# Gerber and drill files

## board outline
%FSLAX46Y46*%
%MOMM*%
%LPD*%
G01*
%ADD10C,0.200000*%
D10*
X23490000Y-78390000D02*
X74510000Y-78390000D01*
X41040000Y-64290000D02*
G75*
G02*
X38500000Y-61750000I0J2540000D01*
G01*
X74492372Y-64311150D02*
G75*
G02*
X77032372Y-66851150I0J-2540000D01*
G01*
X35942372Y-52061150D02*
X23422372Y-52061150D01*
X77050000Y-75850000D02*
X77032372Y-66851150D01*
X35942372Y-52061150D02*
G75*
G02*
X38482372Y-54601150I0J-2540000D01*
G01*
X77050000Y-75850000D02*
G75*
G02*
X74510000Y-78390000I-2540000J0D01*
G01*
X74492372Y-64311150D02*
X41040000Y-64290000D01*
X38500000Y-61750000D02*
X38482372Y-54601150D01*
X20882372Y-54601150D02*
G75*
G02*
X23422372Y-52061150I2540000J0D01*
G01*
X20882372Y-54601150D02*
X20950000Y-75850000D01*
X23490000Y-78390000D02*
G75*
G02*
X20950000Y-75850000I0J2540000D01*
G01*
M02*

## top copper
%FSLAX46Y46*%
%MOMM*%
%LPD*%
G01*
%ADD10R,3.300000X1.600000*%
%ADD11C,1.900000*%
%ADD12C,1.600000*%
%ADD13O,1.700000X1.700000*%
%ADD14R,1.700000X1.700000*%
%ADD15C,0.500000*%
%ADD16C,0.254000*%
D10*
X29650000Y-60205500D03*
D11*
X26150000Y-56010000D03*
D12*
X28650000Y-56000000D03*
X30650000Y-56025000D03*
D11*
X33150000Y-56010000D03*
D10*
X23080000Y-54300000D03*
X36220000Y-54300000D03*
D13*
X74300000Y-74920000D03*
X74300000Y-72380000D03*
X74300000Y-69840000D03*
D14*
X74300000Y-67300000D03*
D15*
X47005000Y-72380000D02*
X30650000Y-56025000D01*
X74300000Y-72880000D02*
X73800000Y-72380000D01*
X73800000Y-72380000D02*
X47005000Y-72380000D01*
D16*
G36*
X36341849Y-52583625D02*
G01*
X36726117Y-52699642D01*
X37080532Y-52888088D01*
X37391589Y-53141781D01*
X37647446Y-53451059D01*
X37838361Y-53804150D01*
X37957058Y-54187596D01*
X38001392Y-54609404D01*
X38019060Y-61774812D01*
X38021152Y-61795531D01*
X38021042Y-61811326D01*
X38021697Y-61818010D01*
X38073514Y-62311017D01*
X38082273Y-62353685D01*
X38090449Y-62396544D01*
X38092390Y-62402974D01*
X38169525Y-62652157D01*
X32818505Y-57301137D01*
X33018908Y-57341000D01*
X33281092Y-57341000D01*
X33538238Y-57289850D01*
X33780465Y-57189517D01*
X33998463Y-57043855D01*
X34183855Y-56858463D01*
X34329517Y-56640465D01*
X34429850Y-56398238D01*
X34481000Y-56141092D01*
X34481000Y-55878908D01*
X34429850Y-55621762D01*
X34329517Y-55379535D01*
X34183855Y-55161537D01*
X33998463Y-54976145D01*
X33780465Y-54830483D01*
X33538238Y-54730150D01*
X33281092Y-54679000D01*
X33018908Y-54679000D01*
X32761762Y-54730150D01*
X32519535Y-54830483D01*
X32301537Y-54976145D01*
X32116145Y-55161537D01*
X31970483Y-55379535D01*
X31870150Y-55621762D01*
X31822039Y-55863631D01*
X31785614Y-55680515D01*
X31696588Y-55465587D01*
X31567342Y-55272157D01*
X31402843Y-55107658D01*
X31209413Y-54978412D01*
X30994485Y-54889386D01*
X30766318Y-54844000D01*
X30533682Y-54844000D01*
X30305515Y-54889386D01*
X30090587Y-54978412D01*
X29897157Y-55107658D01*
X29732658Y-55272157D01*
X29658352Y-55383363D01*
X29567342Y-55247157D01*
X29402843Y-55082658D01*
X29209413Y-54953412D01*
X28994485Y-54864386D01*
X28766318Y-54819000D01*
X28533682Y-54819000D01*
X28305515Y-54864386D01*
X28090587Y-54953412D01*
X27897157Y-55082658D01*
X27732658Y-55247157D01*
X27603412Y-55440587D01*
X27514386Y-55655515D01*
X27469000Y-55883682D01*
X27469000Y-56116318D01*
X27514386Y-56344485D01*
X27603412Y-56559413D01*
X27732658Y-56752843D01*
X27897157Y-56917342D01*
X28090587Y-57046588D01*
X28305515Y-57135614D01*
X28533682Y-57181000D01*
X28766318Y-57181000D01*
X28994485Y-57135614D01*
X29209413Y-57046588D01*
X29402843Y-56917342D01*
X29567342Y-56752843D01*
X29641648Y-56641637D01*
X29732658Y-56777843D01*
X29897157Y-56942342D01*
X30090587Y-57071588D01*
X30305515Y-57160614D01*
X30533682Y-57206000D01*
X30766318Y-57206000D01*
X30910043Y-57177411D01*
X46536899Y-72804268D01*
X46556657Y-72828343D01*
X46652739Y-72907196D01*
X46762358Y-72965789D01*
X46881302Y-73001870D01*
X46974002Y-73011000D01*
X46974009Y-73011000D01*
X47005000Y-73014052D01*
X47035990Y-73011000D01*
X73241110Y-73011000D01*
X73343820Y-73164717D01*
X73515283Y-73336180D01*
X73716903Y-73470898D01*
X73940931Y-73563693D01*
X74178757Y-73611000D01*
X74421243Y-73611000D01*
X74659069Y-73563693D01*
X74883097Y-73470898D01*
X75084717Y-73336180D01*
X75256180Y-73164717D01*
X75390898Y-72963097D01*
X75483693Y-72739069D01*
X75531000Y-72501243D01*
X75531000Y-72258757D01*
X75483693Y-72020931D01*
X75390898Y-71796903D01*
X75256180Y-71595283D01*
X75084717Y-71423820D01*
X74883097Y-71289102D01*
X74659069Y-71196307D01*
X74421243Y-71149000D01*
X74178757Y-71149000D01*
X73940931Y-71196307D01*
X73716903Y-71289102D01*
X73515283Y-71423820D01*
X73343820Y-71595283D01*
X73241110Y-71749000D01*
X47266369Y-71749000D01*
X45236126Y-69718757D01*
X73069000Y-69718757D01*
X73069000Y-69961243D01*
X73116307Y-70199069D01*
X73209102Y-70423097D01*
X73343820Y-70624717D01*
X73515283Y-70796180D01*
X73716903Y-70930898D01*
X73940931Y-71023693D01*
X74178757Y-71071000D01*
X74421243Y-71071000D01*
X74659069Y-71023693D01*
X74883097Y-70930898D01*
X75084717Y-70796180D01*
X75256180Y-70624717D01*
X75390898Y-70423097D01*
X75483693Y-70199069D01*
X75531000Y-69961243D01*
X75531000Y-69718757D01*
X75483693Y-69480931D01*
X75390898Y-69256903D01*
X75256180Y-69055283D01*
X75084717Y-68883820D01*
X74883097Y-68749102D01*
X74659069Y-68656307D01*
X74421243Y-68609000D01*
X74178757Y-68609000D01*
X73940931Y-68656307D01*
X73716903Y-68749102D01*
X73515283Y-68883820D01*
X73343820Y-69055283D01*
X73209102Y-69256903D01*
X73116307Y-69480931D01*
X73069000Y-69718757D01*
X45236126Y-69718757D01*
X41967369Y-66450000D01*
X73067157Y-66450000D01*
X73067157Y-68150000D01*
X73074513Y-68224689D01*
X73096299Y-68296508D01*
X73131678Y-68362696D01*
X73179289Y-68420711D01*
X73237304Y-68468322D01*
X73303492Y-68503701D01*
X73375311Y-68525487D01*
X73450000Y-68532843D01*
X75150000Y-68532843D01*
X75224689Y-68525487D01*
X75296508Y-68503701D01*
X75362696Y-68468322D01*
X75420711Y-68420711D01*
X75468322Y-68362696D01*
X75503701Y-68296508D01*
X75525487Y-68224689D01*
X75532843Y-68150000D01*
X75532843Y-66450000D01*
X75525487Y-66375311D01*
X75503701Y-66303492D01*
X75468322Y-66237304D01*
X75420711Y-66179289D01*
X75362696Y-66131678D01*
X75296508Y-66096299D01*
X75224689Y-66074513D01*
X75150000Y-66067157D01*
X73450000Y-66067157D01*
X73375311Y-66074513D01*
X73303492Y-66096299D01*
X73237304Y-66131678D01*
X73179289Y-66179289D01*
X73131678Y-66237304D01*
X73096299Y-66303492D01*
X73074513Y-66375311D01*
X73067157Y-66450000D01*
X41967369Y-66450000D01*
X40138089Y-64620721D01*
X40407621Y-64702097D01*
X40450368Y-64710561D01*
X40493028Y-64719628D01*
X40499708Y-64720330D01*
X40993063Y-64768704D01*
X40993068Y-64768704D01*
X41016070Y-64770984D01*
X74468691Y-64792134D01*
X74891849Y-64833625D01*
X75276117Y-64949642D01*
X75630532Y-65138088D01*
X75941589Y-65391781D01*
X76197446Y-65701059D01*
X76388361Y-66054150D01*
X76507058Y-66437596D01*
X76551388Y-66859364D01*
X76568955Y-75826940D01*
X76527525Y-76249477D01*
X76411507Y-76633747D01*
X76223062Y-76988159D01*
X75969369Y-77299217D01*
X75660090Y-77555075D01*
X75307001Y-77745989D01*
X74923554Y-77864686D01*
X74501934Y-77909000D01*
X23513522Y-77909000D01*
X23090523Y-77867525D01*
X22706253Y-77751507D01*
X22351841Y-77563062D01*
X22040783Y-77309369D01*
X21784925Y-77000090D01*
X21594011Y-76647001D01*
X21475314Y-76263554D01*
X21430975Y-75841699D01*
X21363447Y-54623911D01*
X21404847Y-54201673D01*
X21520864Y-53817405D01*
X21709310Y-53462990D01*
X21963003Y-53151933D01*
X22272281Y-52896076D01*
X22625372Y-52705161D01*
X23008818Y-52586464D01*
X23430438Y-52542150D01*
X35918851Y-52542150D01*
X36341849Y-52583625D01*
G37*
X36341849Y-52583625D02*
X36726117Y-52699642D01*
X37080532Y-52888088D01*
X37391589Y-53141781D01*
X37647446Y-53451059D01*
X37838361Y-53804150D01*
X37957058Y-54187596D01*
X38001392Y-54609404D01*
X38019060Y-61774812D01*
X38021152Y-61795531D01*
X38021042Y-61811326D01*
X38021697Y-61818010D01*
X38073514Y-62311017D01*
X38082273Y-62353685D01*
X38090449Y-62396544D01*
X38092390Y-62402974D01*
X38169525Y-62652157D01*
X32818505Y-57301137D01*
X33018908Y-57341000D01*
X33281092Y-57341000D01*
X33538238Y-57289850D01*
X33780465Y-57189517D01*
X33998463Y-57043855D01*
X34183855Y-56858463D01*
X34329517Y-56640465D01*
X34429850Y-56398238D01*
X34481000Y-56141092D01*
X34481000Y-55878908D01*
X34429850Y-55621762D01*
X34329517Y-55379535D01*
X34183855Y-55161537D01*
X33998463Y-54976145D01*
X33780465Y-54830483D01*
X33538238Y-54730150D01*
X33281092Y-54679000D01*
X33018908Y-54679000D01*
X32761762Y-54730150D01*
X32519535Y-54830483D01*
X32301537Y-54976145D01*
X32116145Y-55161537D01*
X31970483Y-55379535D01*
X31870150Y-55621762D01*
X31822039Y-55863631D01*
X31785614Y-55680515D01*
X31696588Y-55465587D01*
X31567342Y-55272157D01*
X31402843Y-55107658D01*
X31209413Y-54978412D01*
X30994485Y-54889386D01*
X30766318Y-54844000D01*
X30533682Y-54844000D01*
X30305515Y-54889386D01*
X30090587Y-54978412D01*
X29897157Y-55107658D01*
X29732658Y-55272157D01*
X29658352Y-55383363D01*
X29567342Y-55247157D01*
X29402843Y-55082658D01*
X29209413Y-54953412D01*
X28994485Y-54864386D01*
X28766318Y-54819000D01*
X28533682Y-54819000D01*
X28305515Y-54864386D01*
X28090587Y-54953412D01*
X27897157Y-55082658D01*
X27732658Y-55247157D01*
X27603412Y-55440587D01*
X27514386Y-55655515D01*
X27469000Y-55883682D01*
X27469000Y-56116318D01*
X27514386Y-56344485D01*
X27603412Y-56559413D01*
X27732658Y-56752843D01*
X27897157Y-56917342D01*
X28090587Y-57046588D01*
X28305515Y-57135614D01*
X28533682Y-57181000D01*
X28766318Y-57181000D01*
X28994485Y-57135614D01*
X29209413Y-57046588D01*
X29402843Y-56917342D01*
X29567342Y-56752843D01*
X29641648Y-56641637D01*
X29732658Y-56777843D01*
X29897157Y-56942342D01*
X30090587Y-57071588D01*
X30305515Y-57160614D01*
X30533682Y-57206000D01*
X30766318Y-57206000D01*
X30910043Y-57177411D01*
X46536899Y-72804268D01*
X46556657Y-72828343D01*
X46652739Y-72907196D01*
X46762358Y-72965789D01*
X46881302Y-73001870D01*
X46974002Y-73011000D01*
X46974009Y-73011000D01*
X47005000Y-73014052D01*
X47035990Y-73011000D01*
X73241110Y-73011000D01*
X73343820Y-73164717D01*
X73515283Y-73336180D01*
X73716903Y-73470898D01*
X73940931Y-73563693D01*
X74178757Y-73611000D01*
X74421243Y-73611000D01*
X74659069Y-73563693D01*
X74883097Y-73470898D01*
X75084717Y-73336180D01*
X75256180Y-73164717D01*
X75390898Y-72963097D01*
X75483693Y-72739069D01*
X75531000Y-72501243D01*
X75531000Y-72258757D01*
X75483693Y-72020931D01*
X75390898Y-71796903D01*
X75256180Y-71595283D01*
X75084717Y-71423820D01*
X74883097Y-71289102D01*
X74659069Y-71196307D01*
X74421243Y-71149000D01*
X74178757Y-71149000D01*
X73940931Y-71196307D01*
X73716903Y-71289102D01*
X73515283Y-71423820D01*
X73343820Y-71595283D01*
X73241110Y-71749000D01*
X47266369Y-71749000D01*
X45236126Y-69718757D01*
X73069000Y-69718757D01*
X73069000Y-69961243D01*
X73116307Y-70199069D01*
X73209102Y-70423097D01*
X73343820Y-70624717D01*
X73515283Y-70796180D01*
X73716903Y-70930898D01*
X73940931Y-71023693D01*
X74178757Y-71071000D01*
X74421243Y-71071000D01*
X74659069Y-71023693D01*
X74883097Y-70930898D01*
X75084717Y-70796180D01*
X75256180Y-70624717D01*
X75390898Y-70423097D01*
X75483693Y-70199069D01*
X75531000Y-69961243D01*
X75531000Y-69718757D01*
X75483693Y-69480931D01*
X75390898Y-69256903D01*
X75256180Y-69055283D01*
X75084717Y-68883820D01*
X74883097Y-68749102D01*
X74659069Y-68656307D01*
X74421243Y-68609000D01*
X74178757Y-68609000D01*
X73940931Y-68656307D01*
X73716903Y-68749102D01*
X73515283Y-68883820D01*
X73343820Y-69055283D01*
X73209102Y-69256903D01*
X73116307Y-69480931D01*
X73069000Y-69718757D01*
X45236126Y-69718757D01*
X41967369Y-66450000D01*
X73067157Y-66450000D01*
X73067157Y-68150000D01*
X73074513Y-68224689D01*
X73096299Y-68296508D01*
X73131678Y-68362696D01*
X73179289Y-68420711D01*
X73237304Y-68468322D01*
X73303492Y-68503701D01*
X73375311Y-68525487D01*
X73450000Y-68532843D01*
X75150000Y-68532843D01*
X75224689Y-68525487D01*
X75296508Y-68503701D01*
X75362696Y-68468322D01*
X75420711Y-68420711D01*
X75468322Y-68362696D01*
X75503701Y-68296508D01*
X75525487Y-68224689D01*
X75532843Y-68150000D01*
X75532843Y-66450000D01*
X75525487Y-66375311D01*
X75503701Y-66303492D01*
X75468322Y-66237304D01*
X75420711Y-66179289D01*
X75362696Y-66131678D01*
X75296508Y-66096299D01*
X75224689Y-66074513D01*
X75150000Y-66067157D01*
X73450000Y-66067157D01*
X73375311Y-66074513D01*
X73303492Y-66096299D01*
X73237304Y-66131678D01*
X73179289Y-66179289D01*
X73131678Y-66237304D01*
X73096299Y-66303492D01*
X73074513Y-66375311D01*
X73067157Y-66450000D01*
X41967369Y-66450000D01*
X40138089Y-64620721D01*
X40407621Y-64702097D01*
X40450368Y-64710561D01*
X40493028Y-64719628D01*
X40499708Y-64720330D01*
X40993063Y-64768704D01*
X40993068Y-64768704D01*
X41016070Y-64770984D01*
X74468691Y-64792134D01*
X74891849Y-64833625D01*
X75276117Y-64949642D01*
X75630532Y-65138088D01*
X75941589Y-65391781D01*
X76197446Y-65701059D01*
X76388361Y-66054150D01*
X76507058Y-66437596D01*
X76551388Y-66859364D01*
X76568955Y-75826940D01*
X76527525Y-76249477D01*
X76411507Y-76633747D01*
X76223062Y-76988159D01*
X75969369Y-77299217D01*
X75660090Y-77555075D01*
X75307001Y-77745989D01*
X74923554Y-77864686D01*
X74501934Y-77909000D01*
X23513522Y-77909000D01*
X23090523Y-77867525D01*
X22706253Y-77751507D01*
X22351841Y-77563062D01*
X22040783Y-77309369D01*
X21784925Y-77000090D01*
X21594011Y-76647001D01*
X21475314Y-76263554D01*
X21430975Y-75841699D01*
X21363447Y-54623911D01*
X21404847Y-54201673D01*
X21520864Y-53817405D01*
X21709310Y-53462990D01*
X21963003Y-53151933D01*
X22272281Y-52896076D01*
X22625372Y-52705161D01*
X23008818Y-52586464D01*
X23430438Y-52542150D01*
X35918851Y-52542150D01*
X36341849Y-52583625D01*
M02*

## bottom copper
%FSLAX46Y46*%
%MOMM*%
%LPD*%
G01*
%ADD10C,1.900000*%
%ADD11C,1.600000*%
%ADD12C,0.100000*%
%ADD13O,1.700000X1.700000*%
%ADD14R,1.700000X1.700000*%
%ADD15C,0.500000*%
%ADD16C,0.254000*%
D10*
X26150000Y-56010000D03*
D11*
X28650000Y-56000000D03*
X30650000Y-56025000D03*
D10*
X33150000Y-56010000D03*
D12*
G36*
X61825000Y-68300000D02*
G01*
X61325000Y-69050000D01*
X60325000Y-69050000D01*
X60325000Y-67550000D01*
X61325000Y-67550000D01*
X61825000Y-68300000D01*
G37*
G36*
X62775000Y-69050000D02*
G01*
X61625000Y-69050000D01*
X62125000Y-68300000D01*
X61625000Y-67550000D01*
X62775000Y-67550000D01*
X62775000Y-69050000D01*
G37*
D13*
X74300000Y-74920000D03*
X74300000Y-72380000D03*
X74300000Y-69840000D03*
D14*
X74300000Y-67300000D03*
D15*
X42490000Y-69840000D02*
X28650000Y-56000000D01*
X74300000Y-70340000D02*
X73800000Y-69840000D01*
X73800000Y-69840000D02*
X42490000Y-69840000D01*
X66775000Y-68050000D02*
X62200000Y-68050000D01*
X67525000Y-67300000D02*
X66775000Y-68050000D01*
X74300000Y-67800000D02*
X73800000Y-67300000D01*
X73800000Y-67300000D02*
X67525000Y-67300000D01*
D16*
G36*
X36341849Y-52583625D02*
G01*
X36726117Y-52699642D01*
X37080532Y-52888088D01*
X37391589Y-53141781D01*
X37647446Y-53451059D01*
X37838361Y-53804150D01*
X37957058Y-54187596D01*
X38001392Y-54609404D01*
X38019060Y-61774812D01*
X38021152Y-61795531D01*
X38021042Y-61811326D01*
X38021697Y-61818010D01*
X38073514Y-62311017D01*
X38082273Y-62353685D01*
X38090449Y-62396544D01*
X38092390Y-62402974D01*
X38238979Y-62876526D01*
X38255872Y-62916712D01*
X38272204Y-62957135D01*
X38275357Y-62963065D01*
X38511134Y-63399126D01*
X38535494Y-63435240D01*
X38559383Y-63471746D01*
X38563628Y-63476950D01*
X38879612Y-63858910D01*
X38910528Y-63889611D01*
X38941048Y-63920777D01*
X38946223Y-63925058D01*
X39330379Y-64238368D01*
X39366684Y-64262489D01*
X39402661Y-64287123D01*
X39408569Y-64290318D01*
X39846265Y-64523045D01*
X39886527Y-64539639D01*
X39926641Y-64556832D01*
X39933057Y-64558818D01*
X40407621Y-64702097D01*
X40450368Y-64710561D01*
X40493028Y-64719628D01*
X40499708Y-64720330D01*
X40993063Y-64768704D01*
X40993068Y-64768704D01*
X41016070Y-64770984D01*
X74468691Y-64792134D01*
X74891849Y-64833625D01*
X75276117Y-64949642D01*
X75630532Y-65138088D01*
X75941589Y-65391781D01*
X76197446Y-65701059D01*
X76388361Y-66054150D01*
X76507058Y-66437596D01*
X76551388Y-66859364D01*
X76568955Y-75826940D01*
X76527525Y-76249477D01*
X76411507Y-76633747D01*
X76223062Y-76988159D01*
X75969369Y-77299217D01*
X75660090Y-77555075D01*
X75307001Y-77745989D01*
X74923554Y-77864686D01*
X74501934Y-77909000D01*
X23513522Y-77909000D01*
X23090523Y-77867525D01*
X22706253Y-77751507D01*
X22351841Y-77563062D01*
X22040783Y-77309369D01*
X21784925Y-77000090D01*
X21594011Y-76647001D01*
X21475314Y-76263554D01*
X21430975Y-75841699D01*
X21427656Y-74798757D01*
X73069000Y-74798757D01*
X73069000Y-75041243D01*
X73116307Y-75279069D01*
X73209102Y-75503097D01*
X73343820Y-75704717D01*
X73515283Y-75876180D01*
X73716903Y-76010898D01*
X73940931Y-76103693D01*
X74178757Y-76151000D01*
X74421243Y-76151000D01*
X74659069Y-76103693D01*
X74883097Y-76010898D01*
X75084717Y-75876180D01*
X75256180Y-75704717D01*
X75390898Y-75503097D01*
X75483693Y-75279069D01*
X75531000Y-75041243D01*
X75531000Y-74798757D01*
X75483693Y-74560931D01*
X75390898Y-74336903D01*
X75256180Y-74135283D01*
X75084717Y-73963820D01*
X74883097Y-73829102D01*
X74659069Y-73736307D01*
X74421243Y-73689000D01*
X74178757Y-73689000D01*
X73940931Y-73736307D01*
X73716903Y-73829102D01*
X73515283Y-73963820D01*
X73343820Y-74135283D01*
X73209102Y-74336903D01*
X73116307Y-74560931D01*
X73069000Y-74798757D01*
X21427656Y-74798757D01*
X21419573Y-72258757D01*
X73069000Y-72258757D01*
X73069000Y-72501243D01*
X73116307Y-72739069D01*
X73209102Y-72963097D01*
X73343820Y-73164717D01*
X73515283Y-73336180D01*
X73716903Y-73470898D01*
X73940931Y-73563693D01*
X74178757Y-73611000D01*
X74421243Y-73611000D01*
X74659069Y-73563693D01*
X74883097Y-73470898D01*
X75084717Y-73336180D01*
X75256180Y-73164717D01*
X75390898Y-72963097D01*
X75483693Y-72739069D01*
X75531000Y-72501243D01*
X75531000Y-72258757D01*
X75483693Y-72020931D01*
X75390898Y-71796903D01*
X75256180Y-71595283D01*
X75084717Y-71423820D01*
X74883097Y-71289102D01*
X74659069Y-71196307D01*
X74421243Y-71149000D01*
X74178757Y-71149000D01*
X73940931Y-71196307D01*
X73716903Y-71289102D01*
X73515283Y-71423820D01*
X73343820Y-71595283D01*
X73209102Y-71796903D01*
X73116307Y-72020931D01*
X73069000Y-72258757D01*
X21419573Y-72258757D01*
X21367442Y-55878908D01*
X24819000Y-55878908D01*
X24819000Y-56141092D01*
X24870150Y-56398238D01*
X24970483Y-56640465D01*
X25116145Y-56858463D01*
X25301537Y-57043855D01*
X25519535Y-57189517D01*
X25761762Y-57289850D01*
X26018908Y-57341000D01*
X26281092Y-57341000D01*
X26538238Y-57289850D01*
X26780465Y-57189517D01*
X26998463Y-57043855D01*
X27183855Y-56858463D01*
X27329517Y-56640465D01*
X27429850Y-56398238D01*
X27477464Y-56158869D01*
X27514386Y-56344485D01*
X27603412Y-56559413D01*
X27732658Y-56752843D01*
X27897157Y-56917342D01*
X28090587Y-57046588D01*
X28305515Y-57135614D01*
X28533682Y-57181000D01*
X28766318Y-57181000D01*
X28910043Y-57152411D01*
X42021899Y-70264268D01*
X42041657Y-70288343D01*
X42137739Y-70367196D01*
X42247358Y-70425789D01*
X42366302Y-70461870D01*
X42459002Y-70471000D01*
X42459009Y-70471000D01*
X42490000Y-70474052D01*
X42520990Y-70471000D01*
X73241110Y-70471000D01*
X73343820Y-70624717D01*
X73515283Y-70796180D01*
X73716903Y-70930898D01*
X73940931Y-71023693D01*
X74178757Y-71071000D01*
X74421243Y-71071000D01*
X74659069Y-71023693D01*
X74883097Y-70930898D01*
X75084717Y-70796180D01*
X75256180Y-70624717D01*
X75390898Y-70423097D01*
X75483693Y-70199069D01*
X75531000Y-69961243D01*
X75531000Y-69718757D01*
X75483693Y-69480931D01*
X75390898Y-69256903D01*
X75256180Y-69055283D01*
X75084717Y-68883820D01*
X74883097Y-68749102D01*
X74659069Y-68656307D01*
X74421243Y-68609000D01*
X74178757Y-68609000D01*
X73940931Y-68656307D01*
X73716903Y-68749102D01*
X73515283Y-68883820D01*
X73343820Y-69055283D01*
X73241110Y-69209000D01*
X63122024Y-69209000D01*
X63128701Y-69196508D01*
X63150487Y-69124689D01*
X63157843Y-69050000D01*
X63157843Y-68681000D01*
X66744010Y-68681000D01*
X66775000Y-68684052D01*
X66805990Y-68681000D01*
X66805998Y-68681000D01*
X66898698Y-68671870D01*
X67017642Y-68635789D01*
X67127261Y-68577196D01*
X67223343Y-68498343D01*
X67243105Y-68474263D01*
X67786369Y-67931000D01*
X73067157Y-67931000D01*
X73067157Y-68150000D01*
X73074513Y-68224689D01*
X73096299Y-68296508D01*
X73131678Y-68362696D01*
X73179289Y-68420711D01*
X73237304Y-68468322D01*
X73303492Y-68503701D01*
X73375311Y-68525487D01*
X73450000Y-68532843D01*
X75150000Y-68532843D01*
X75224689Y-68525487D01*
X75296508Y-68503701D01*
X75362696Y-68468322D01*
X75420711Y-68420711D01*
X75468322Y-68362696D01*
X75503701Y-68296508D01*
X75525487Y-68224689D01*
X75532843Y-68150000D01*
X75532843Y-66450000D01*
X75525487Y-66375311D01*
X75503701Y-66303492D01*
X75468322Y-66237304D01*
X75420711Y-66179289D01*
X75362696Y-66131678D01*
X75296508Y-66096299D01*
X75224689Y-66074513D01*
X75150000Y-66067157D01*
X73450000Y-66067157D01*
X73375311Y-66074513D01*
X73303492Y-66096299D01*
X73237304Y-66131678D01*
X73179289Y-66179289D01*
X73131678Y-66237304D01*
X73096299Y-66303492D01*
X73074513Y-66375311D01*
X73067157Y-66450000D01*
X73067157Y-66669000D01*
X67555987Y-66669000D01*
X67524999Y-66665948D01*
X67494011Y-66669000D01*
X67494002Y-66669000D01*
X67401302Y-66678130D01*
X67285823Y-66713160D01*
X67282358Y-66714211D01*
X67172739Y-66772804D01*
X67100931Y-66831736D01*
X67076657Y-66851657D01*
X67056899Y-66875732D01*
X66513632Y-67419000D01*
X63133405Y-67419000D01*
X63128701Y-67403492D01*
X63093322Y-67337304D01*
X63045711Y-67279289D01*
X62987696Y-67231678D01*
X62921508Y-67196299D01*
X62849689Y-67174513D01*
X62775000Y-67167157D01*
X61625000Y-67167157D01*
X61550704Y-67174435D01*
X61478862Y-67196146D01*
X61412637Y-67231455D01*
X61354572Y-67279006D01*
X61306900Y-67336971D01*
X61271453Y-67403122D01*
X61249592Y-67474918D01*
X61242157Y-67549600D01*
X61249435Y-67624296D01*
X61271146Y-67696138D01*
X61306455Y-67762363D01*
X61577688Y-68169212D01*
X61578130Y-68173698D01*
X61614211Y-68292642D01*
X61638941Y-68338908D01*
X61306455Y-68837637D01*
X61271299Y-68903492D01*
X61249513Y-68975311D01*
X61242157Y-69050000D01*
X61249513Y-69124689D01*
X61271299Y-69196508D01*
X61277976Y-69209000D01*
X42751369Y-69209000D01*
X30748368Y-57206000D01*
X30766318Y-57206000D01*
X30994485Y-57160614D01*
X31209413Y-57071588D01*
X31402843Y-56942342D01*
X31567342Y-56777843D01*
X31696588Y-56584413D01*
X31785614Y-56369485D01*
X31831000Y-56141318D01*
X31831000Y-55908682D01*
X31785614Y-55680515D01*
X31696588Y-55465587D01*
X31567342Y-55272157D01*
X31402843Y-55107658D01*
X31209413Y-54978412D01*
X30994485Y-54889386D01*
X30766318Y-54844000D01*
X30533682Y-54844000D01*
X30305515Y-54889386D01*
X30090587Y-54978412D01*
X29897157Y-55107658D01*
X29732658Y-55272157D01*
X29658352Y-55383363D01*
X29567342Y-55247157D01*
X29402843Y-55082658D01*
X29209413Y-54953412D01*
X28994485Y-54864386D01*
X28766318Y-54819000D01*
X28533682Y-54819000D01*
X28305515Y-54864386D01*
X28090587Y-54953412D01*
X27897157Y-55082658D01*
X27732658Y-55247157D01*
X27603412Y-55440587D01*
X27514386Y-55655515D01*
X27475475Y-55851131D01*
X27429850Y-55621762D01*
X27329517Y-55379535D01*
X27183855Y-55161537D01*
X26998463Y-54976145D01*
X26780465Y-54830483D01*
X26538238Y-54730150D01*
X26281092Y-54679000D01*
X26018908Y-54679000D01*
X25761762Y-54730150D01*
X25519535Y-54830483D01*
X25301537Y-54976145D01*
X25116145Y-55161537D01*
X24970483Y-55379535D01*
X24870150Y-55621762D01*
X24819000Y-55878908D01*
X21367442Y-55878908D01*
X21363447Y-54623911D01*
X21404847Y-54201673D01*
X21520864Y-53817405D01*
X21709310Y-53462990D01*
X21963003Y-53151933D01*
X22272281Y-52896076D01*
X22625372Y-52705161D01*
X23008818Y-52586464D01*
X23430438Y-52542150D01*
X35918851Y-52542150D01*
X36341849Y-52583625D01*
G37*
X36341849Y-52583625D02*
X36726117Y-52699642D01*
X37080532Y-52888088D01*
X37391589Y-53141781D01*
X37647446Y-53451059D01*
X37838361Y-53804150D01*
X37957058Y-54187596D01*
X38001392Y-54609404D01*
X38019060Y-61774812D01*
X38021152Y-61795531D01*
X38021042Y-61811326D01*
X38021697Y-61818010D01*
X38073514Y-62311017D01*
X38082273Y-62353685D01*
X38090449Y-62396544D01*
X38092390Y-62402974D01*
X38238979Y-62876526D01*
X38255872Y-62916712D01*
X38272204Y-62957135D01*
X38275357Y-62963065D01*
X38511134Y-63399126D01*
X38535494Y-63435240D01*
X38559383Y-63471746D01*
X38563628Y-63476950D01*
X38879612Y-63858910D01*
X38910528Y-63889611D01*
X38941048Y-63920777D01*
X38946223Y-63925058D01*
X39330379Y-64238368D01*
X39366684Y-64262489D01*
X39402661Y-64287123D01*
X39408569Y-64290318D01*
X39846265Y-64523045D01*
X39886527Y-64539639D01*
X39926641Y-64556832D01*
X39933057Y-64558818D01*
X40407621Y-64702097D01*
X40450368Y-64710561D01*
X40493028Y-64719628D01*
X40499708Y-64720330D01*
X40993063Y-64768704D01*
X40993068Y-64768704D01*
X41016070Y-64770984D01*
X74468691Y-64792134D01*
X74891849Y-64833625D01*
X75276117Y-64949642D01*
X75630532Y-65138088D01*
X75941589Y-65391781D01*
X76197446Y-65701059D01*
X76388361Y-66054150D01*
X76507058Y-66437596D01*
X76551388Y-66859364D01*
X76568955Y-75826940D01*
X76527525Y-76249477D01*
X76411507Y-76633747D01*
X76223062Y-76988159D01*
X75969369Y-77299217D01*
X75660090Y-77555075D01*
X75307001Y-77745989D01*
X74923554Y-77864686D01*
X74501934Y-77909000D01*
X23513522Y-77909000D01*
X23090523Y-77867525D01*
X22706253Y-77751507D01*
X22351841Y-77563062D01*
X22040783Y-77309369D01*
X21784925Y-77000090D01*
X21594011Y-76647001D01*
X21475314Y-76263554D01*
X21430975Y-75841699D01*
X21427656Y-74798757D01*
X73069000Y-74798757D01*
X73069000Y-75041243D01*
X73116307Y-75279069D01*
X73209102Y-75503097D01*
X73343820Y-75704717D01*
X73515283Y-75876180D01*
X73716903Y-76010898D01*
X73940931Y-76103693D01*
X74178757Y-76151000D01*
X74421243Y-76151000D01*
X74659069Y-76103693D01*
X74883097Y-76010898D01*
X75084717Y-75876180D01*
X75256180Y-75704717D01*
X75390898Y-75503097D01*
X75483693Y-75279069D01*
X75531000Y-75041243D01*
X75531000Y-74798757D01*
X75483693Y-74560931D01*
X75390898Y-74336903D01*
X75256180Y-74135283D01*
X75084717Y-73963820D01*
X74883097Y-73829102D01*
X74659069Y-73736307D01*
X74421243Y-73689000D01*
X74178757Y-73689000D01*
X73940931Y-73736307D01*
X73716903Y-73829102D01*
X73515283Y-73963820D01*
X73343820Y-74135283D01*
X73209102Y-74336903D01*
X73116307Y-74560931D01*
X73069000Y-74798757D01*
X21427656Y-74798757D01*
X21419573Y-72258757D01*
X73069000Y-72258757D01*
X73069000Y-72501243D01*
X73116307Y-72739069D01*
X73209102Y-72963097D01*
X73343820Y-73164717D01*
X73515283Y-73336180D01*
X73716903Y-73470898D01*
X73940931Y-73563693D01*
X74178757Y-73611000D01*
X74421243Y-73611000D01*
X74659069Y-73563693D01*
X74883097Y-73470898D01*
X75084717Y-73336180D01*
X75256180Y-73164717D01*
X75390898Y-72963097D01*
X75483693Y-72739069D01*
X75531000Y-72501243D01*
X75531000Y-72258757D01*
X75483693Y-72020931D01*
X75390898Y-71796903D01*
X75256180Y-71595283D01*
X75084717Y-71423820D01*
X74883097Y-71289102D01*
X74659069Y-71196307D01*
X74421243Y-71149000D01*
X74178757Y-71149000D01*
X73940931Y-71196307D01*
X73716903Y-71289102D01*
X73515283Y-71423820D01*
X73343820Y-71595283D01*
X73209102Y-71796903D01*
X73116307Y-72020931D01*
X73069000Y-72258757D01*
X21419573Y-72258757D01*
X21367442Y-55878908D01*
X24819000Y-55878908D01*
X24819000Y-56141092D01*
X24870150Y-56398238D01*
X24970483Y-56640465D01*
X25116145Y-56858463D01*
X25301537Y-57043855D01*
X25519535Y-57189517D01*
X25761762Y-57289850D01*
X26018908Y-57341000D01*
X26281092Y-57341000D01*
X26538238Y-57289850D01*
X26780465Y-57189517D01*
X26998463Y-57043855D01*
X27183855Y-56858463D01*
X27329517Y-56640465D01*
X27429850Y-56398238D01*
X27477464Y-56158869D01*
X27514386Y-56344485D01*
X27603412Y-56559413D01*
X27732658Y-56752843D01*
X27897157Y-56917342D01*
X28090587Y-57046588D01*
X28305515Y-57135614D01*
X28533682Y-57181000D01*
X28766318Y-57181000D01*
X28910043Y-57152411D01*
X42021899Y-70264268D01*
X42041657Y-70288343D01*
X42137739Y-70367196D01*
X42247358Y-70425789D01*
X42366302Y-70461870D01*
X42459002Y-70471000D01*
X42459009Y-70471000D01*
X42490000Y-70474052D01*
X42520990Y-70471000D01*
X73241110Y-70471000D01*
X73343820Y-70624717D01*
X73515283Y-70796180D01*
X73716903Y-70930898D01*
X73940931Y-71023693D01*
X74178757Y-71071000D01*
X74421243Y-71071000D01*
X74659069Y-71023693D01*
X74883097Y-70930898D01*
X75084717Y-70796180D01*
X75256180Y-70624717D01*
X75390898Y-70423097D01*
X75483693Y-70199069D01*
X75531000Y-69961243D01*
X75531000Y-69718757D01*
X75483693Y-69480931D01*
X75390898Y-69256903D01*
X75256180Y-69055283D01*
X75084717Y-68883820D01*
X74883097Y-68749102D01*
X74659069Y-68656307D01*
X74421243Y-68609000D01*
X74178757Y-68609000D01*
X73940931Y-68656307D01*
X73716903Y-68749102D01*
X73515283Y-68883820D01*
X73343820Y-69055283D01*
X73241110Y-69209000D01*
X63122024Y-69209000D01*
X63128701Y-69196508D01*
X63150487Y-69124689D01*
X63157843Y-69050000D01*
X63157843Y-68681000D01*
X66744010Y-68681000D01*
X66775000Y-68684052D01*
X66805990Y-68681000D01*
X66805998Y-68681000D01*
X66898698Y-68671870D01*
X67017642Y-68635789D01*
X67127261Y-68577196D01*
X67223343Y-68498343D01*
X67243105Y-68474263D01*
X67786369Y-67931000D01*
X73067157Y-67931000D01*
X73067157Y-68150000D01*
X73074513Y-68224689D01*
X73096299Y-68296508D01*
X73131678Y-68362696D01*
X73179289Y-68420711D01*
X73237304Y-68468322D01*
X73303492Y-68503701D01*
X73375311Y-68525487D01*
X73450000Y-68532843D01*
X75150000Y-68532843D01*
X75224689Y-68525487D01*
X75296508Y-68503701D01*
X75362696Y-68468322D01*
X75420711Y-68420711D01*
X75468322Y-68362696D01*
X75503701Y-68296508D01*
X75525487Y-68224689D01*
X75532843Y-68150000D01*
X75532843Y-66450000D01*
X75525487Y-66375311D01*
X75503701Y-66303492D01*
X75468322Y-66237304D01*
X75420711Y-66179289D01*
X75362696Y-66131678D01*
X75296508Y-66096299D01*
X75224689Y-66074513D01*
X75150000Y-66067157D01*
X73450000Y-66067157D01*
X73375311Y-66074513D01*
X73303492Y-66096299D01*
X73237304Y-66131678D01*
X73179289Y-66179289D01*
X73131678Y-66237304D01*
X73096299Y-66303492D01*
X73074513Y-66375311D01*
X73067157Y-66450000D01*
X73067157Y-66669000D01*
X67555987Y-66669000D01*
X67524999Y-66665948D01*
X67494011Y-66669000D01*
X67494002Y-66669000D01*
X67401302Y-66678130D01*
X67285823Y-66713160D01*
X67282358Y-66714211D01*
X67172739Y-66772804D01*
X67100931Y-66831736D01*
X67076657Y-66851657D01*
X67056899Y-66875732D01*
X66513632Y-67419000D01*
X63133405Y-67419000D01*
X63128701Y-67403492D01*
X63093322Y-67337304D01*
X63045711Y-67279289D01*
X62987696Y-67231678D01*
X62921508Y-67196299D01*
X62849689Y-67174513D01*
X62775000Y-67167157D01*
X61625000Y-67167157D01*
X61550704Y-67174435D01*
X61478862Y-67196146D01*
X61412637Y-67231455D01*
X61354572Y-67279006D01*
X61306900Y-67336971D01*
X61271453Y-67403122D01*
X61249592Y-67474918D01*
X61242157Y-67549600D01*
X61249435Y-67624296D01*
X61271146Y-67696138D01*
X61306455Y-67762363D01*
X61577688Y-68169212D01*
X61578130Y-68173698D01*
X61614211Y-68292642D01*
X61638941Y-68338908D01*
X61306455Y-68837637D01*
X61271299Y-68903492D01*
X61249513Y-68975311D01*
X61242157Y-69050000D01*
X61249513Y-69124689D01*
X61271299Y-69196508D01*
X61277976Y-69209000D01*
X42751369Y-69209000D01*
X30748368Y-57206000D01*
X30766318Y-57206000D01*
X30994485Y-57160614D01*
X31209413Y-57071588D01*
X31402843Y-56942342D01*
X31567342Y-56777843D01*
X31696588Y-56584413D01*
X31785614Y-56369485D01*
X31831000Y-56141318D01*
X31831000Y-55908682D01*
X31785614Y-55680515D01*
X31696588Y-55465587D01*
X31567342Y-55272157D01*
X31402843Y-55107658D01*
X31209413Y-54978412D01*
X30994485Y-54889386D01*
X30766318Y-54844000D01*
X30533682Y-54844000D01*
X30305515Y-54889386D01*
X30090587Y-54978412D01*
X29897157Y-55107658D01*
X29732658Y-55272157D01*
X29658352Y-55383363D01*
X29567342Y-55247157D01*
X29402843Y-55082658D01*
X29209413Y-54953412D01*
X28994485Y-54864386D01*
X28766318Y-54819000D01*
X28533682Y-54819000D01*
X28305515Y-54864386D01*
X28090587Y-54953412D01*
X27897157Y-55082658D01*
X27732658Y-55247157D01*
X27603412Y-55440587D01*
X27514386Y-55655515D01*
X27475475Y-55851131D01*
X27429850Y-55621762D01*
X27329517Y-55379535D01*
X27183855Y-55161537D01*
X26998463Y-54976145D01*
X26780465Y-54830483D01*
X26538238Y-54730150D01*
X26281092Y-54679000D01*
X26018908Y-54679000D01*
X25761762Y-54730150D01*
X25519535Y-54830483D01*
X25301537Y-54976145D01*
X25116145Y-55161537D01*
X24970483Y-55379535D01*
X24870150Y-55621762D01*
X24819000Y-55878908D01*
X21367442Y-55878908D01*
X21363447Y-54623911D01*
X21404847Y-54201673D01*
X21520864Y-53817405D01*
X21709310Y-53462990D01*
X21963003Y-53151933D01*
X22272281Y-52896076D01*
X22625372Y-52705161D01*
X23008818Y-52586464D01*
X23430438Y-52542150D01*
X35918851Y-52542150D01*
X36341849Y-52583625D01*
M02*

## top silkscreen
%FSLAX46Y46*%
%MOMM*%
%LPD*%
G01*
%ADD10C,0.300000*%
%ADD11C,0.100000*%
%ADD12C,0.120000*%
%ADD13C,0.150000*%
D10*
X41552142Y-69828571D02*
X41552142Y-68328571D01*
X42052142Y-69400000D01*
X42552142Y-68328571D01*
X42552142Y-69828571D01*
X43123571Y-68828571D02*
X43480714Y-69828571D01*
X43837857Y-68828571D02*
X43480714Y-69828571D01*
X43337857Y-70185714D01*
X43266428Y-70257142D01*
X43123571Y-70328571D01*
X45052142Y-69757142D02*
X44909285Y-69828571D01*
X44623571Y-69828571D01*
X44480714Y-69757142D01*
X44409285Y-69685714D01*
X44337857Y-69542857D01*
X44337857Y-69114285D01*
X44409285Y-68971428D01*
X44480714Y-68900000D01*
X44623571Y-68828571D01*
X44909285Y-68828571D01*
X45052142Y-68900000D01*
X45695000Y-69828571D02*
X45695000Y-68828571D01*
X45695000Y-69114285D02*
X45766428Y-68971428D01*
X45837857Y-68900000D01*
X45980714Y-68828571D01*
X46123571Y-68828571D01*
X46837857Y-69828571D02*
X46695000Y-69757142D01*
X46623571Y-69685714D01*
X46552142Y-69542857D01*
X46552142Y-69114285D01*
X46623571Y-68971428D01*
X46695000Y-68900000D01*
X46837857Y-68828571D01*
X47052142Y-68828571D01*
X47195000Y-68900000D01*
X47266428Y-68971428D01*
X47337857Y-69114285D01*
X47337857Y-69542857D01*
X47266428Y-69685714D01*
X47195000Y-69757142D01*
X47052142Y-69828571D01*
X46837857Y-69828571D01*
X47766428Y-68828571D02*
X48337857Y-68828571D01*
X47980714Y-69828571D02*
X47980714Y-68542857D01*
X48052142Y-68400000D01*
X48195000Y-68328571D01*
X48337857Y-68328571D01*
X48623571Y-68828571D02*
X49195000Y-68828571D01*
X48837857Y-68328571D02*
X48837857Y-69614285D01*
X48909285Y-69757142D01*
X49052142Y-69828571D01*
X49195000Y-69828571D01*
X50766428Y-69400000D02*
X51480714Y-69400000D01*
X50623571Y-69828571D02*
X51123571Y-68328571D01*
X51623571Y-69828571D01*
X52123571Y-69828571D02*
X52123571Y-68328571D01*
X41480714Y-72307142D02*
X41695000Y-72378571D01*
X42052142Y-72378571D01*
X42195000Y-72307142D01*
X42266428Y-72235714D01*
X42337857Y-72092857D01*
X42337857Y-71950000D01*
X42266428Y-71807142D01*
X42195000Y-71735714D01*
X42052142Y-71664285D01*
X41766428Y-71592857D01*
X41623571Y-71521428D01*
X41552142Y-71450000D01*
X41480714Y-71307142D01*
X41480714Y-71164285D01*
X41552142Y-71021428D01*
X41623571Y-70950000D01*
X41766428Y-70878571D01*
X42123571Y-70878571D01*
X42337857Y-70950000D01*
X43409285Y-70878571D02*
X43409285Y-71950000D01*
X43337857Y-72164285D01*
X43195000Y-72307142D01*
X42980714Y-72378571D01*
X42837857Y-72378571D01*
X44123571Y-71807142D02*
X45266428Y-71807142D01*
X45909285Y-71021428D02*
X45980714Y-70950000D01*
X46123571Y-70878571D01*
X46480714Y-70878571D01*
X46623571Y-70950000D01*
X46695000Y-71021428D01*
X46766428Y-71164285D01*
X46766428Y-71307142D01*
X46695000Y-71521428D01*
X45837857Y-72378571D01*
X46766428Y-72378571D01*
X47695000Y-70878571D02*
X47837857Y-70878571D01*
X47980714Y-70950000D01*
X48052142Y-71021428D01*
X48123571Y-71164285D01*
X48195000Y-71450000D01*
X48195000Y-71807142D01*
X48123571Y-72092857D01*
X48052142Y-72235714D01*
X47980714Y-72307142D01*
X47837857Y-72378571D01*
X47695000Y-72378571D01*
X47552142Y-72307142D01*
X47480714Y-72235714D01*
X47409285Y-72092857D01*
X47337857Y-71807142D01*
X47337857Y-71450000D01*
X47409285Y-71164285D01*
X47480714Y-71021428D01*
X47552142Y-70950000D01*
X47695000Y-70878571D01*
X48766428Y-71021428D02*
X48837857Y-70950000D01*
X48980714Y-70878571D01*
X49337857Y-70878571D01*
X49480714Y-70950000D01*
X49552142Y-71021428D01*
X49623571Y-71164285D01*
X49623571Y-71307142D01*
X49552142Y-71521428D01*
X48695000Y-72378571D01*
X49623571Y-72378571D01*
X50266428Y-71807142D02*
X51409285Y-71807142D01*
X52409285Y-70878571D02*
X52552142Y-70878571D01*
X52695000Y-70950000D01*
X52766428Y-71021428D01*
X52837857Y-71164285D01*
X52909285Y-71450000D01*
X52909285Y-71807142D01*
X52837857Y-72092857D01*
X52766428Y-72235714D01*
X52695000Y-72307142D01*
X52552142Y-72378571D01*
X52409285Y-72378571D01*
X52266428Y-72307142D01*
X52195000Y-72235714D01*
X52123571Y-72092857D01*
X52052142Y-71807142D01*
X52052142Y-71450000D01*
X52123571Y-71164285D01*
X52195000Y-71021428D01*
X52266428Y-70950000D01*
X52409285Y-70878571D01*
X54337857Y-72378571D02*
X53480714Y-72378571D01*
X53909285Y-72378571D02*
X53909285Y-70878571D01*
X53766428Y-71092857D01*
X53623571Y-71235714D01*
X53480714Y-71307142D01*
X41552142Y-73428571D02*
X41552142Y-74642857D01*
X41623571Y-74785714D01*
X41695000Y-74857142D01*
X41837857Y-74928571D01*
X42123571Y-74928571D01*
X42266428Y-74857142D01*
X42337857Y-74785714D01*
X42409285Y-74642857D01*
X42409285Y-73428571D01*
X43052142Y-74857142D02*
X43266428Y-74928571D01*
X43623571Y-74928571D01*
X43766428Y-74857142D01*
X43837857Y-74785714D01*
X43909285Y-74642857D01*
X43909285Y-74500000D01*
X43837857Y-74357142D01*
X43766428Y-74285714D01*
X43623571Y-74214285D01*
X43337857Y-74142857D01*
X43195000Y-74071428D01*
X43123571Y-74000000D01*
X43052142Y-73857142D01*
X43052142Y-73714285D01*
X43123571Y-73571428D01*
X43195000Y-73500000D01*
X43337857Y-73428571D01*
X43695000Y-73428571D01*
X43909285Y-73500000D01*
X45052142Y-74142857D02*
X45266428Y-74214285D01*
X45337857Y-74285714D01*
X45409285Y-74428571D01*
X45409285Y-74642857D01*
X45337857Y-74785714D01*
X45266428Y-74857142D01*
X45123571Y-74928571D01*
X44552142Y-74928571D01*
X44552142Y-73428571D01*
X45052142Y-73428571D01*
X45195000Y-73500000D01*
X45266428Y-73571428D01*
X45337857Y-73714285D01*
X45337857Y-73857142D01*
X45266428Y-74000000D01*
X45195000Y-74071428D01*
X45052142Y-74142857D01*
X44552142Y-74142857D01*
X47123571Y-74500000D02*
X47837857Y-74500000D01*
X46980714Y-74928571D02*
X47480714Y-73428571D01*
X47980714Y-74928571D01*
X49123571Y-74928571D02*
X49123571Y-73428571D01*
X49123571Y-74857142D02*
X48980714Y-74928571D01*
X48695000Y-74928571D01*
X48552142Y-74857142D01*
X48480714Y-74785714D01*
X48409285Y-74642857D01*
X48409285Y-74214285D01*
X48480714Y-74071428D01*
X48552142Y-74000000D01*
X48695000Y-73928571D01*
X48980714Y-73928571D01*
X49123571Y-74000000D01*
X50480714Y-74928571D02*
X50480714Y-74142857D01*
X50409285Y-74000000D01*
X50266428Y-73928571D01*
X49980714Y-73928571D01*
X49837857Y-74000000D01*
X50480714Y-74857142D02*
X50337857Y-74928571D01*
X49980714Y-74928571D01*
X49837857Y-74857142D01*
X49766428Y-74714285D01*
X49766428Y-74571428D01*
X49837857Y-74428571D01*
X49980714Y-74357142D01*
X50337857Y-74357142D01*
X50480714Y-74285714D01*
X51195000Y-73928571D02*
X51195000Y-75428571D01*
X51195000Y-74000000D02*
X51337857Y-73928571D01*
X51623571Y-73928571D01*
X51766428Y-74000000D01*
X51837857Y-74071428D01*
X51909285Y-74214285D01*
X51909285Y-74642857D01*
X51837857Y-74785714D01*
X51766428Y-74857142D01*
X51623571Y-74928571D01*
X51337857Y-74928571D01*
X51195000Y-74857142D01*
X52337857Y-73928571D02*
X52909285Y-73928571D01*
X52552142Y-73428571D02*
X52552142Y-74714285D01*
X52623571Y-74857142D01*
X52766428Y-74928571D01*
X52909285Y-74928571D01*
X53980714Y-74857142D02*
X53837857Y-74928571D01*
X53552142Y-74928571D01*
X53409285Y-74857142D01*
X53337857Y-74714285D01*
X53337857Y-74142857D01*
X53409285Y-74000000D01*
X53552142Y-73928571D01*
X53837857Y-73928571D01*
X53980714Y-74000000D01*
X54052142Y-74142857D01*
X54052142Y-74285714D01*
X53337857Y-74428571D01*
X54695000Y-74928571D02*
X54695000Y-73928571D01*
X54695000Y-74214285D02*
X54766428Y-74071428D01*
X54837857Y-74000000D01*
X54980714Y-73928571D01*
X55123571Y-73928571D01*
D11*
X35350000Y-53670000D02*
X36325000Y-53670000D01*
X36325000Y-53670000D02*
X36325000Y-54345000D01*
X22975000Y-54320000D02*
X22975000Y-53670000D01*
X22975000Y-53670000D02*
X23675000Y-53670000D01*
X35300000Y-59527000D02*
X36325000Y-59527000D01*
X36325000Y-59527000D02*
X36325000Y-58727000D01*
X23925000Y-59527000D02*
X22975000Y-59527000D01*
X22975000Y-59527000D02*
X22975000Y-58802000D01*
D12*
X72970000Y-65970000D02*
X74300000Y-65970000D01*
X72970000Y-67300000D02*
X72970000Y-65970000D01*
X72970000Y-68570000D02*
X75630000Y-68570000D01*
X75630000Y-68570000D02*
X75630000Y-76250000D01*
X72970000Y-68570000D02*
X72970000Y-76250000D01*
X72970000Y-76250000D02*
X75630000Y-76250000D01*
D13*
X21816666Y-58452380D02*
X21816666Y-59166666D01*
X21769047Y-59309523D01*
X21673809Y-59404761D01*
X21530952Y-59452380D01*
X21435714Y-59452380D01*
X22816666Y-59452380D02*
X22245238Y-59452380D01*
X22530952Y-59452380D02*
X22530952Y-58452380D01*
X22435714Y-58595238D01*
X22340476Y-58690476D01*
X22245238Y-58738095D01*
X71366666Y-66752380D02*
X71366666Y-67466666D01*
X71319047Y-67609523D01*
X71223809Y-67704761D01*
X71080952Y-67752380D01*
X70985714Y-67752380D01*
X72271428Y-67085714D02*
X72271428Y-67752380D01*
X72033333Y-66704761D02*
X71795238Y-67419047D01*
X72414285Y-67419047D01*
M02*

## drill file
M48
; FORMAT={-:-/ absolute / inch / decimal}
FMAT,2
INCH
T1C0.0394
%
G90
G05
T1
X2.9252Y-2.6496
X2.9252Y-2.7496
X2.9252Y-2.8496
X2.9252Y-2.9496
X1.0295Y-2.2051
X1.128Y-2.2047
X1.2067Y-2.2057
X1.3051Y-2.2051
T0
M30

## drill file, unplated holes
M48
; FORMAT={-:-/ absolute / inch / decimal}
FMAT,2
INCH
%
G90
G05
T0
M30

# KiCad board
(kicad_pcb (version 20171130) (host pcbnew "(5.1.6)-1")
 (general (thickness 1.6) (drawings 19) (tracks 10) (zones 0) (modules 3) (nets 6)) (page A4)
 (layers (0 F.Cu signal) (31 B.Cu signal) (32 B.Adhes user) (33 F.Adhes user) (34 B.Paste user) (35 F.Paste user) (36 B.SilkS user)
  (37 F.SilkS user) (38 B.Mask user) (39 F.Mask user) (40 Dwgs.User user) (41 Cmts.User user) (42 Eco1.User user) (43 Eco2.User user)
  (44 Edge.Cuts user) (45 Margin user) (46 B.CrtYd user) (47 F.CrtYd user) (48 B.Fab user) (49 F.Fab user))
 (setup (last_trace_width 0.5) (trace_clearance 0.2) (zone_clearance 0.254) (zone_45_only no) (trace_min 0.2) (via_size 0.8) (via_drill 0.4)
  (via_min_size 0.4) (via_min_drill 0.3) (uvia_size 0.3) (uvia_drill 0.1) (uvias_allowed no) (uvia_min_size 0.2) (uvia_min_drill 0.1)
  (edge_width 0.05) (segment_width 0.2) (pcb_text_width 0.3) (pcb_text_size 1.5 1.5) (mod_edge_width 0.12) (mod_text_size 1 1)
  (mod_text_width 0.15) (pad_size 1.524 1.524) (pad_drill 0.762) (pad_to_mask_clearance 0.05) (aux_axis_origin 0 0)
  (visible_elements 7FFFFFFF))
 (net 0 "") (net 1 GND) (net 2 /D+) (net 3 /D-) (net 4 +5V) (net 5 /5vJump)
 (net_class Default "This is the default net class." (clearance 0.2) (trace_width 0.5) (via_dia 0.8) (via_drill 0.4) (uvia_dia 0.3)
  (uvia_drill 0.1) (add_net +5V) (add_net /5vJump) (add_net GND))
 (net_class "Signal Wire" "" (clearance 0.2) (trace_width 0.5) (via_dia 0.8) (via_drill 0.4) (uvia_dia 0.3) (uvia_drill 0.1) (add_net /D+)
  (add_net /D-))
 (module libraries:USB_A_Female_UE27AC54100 (layer F.Cu) (at 29.65 53.3 180)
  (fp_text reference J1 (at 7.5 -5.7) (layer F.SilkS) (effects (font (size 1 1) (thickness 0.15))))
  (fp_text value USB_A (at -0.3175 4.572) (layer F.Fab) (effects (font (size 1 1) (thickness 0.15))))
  (fp_line (start -5.7 -0.37) (end -6.675 -0.37) (layer F.SilkS) (width 0.1))
  (fp_line (start -6.675 -0.37) (end -6.675 -1.045) (layer F.SilkS) (width 0.1))
  (fp_line (start 6.675 -1.02) (end 6.675 -0.37) (layer F.SilkS) (width 0.1))
  (fp_line (start 6.675 -0.37) (end 5.975 -0.37) (layer F.SilkS) (width 0.1))
  (fp_line (start -5.65 -6.227) (end -6.675 -6.227) (layer F.SilkS) (width 0.1))
  (fp_line (start -6.675 -6.227) (end -6.675 -5.427) (layer F.SilkS) (width 0.1))
  (fp_line (start 5.725 -6.227) (end 6.675 -6.227) (layer F.SilkS) (width 0.1))
  (fp_line (start 6.675 -6.227) (end 6.675 -5.502) (layer F.SilkS) (width 0.1))
  (pad 5 smd rect (at 0 -6.9055 180) (size 3.3 1.6) (layers F.Cu F.Paste F.Mask) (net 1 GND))
  (pad 4 thru_hole circle (at 3.5 -2.71 180) (size 1.9 1.9) (drill 1) (layers *.Cu *.Mask) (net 1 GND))
  (pad 3 thru_hole circle (at 1 -2.7 180) (size 1.6 1.6) (drill 1) (layers *.Cu *.Mask) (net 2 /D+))
  (pad 2 thru_hole circle (at -1 -2.725 180) (size 1.6 1.6) (drill 1) (layers *.Cu *.Mask) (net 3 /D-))
  (pad 1 thru_hole circle (at -3.5 -2.71 180) (size 1.9 1.9) (drill 1) (layers *.Cu *.Mask) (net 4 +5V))
  (pad 5 smd rect (at 6.57 -1 180) (size 3.3 1.6) (layers F.Cu F.Paste F.Mask) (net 1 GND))
  (pad 5 smd rect (at -6.57 -1 180) (size 3.3 1.6) (layers F.Cu F.Paste F.Mask) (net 1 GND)))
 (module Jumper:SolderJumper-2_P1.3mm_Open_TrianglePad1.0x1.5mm (layer B.Cu) (at 61.55 68.3)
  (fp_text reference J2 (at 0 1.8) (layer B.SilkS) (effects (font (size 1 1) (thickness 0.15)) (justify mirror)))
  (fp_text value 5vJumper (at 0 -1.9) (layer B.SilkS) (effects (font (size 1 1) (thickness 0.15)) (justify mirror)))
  (pad 1 smd custom (at -0.725 0) (size 0.3 0.3) (layers B.Cu B.Mask) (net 4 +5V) (zone_connect 2)
   (options (clearance outline) (anchor rect)) (primitives))
  (pad 2 smd custom (at 0.725 0) (size 0.3 0.3) (layers B.Cu B.Mask) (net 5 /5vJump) (zone_connect 2)
   (options (clearance outline) (anchor rect)) (primitives)))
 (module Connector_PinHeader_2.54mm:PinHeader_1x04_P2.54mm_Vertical (layer F.Cu) (at 74.3 67.3)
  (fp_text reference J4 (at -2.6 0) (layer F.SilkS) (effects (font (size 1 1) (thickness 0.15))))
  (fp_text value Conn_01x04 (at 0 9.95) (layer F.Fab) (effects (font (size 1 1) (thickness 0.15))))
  (fp_line (start -1.33 -1.33) (end 0 -1.33) (layer F.SilkS) (width 0.12))
  (fp_line (start -1.33 0) (end -1.33 -1.33) (layer F.SilkS) (width 0.12))
  (fp_line (start -1.33 1.27) (end 1.33 1.27) (layer F.SilkS) (width 0.12))
  (fp_line (start 1.33 1.27) (end 1.33 8.95) (layer F.SilkS) (width 0.12))
  (fp_line (start -1.33 1.27) (end -1.33 8.95) (layer F.SilkS) (width 0.12))
  (fp_line (start -1.33 8.95) (end 1.33 8.95) (layer F.SilkS) (width 0.12))
  (pad 4 thru_hole oval (at 0 7.62) (size 1.7 1.7) (drill 1) (layers *.Cu *.Mask) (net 1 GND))
  (pad 3 thru_hole oval (at 0 5.08) (size 1.7 1.7) (drill 1) (layers *.Cu *.Mask) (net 3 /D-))
  (pad 2 thru_hole oval (at 0 2.54) (size 1.7 1.7) (drill 1) (layers *.Cu *.Mask) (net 2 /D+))
  (pad 1 thru_hole rect (at 0 0) (size 1.7 1.7) (drill 1) (layers *.Cu *.Mask) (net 5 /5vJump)))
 (gr_line (start 23.49 78.39) (end 74.51 78.39) (layer Edge.Cuts) (width 0.2))
 (gr_arc (start 41.04 61.75) (end 38.5 61.75) (angle -90) (layer Edge.Cuts) (width 0.2))
 (gr_arc (start 74.492372 66.85115) (end 77.032372 66.85115) (angle -90) (layer Edge.Cuts) (width 0.2))
 (gr_line (start 35.942372 52.06115) (end 23.422372 52.06115) (layer Edge.Cuts) (width 0.2))
 (gr_line (start 77.05 75.85) (end 77.032372 66.85115) (layer Edge.Cuts) (width 0.2))
 (gr_arc (start 35.942372 54.60115) (end 38.482372 54.60115) (angle -90) (layer Edge.Cuts) (width 0.2))
 (gr_arc (start 74.51 75.85) (end 74.51 78.39) (angle -90) (layer Edge.Cuts) (width 0.2))
 (gr_line (start 74.492372 64.31115) (end 41.04 64.29) (layer Edge.Cuts) (width 0.2))
 (gr_line (start 38.5 61.75) (end 38.482372 54.60115) (layer Edge.Cuts) (width 0.2))
 (gr_arc (start 23.422372 54.60115) (end 23.422372 52.06115) (angle -90) (layer Edge.Cuts) (width 0.2))
 (gr_line (start 20.882372 54.60115) (end 20.95 75.85) (layer Edge.Cuts) (width 0.2))
 (gr_arc (start 23.49 75.85) (end 20.95 75.85) (angle -90) (layer Edge.Cuts) (width 0.2))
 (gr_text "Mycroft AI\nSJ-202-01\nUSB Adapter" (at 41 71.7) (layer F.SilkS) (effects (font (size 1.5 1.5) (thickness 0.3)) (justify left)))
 (segment (start 42.49 69.84) (end 28.65 56) (width 0.5) (layer B.Cu) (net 2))
 (segment (start 74.3 70.34) (end 73.8 69.84) (width 0.5) (layer B.Cu) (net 2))
 (segment (start 73.8 69.84) (end 42.49 69.84) (width 0.5) (layer B.Cu) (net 2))
 (segment (start 47.005 72.38) (end 30.65 56.025) (width 0.5) (layer F.Cu) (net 3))
 (segment (start 74.3 72.88) (end 73.8 72.38) (width 0.5) (layer F.Cu) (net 3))
 (segment (start 73.8 72.38) (end 47.005 72.38) (width 0.5) (layer F.Cu) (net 3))
 (segment (start 66.775 68.05) (end 62.2 68.05) (width 0.5) (layer B.Cu) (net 5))
 (segment (start 67.525 67.3) (end 66.775 68.05) (width 0.5) (layer B.Cu) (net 5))
 (segment (start 74.3 67.8) (end 73.8 67.3) (width 0.5) (layer B.Cu) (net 5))
 (segment (start 73.8 67.3) (end 67.525 67.3) (width 0.5) (layer B.Cu) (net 5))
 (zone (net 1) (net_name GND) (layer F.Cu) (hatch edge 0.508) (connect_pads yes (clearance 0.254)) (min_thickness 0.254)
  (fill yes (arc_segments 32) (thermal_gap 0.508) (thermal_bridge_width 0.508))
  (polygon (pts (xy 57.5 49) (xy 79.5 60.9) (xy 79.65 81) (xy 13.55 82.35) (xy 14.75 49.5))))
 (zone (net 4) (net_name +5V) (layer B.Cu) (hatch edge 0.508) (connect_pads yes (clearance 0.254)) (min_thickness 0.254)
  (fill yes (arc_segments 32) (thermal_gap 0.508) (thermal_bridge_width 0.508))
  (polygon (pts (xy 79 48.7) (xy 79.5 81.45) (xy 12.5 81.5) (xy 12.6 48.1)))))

